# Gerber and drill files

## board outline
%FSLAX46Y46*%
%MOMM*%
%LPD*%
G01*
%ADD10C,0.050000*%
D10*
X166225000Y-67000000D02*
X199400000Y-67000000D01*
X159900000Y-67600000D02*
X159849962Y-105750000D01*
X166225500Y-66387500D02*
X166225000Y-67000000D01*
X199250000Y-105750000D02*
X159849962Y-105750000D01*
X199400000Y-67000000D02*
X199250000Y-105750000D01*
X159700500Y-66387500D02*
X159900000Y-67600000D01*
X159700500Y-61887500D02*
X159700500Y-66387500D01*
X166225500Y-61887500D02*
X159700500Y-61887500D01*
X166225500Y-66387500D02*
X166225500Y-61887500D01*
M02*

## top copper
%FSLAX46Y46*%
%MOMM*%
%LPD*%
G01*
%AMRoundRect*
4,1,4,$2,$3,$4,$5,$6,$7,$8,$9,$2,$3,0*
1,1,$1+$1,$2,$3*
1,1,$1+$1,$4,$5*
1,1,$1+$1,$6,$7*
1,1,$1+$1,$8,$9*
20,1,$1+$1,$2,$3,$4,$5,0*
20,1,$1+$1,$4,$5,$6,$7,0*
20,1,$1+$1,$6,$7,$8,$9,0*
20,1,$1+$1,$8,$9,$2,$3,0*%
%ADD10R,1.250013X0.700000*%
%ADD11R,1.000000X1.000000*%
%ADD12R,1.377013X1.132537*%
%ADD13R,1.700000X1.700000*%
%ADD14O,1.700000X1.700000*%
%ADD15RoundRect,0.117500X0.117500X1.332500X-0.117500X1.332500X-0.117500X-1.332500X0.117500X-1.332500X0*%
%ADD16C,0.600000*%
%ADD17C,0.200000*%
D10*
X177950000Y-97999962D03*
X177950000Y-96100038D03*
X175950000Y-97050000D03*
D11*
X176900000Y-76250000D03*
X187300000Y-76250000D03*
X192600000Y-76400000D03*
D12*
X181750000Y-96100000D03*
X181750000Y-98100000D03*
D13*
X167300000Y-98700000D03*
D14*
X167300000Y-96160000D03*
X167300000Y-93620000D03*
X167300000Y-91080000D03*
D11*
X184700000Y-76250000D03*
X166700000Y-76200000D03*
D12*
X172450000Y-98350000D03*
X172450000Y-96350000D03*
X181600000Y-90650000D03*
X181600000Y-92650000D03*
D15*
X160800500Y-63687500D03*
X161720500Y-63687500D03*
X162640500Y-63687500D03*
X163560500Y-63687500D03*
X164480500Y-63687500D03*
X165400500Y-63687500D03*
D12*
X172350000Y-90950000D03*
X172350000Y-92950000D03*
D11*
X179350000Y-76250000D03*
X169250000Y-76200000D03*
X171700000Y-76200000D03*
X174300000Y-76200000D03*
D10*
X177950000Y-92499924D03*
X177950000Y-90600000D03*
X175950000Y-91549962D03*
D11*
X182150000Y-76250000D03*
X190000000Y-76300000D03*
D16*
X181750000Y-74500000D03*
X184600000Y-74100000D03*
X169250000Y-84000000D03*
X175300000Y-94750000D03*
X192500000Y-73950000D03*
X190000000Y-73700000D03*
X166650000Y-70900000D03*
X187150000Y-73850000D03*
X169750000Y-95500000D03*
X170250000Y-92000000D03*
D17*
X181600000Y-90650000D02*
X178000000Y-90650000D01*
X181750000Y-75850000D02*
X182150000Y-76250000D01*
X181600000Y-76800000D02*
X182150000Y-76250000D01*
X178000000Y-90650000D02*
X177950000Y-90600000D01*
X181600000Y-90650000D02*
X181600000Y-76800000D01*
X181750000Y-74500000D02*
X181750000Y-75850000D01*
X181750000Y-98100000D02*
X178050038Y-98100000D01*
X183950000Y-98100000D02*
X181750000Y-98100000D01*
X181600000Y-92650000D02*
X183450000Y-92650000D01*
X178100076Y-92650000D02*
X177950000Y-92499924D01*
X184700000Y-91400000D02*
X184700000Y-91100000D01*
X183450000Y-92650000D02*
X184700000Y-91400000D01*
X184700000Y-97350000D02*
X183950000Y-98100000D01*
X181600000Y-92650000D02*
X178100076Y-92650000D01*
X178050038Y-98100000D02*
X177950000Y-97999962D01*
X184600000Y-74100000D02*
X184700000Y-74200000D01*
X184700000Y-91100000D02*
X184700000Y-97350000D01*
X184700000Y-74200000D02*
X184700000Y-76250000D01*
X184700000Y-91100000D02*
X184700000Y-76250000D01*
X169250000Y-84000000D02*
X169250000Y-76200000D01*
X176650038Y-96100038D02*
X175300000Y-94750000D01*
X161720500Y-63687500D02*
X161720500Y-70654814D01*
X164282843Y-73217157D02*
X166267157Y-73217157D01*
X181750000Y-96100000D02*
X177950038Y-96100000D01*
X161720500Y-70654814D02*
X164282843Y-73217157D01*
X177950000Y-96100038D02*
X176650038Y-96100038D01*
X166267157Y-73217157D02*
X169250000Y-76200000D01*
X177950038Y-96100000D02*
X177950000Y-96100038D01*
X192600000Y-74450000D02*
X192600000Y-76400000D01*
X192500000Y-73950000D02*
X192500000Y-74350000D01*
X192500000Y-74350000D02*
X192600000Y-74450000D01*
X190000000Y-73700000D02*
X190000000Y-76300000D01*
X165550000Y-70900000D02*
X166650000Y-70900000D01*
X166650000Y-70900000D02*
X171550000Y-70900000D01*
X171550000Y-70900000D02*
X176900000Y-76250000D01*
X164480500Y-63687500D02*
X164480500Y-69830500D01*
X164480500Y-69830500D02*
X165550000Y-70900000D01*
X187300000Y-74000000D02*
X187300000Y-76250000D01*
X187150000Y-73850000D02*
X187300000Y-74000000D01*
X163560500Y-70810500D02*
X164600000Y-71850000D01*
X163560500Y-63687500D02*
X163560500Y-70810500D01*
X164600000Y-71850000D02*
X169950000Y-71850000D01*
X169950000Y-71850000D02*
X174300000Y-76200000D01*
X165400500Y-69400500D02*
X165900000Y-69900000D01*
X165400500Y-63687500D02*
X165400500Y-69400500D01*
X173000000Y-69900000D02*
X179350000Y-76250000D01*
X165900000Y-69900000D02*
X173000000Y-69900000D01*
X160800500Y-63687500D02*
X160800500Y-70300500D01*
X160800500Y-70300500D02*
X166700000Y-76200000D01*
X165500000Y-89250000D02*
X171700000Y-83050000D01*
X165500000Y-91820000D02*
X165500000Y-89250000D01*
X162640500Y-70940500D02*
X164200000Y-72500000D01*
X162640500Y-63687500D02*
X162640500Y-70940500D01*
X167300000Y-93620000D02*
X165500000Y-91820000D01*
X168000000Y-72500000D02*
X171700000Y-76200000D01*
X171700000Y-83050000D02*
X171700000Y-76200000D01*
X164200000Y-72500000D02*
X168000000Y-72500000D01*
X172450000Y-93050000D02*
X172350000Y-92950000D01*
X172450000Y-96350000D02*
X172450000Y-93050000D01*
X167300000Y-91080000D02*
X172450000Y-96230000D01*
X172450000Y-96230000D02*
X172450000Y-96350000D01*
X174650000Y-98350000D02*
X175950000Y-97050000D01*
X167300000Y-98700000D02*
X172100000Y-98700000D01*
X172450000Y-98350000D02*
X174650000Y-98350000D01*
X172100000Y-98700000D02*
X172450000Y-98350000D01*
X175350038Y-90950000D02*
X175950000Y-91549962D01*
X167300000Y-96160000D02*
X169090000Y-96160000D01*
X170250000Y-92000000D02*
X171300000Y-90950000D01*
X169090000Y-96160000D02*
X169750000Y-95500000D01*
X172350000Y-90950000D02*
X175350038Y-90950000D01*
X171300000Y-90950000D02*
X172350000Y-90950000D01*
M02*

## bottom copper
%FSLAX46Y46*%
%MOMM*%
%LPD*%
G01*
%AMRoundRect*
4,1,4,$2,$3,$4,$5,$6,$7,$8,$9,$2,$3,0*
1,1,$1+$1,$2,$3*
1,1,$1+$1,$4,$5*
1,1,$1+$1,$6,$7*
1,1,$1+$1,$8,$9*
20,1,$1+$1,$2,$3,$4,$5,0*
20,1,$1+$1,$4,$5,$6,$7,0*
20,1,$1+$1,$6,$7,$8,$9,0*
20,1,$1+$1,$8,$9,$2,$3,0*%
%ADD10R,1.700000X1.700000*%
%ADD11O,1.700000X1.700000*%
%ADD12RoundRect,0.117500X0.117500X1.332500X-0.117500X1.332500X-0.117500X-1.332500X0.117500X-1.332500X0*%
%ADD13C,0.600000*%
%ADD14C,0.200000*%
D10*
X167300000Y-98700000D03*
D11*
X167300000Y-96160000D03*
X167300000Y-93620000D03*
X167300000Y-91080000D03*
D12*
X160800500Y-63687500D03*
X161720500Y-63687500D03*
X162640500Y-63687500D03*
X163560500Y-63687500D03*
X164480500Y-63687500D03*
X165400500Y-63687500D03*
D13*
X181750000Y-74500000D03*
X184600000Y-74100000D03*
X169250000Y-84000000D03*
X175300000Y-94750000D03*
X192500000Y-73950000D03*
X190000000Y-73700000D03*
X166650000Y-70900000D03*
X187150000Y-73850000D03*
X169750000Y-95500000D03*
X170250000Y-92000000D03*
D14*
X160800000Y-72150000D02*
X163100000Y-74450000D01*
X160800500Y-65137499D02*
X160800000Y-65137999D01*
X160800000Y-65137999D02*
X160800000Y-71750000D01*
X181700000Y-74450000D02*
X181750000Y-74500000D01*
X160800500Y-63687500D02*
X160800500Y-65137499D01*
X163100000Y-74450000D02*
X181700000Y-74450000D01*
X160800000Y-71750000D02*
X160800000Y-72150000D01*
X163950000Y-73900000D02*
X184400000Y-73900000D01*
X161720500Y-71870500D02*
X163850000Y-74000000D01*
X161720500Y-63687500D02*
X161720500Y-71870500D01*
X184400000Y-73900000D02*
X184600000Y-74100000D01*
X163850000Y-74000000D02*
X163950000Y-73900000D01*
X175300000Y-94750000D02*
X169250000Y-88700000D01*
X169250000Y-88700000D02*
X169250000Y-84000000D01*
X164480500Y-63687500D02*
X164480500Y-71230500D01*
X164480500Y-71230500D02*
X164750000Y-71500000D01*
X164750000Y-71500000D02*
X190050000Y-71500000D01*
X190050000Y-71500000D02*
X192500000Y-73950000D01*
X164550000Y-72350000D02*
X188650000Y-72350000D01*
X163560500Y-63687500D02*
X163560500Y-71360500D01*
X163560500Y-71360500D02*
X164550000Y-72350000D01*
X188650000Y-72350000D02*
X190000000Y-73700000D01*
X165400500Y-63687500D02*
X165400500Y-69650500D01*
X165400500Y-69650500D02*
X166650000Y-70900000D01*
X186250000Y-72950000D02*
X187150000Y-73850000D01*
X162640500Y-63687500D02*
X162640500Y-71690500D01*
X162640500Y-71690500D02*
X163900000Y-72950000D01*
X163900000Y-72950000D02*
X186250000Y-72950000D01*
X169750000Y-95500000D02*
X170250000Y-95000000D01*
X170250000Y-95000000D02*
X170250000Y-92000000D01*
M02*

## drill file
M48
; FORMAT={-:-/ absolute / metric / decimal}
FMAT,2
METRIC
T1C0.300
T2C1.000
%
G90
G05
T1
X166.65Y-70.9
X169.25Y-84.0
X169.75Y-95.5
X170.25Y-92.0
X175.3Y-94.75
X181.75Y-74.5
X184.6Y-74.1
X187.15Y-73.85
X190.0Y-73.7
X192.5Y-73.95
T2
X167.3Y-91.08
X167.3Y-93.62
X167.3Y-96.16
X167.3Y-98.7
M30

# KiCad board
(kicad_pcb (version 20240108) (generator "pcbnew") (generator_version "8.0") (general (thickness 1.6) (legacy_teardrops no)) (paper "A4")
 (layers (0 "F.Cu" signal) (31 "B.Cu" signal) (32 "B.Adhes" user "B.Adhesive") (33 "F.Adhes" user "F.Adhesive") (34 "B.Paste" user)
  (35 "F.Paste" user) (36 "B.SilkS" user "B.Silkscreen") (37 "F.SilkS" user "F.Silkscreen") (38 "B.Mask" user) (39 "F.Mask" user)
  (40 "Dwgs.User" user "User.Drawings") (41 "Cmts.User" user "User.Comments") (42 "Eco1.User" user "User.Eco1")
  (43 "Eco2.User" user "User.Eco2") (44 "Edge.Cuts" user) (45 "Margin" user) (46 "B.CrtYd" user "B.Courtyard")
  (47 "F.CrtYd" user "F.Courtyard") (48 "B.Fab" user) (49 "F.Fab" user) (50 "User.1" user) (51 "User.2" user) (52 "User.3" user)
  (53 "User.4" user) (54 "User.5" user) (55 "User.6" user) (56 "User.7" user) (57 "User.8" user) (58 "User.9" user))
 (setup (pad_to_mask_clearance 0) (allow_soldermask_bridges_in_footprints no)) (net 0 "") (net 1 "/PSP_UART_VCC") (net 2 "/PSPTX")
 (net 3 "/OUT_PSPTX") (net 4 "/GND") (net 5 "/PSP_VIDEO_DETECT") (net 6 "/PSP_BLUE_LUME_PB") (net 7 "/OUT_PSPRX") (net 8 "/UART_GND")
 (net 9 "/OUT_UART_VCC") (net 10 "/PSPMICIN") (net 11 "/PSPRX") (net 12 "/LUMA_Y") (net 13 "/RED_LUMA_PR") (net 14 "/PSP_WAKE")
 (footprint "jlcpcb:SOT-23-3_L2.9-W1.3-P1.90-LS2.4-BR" (layer "F.Cu") (at 176.95 97.05)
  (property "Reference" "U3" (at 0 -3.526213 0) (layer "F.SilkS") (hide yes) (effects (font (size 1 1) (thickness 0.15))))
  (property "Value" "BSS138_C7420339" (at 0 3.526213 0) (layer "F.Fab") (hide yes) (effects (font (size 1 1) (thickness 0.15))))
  (pad "1" smd rect (at 1 0.949962) (size 1.250013 0.7) (layers "F.Cu" "F.Paste" "F.Mask") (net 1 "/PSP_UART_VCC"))
  (pad "2" smd rect (at 1 -0.949962) (size 1.250013 0.7) (layers "F.Cu" "F.Paste" "F.Mask") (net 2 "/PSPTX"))
  (pad "3" smd rect (at -1 0) (size 1.250013 0.7) (layers "F.Cu" "F.Paste" "F.Mask") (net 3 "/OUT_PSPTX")))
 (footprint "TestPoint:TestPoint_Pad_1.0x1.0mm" (layer "F.Cu") (at 176.9 76.25)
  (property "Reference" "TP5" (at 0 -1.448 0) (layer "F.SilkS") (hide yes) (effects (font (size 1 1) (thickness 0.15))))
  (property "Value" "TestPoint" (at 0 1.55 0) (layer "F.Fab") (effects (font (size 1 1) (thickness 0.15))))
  (pad "1" smd rect (at 0 0) (size 1 1) (layers "F.Cu" "F.Mask") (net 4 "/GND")))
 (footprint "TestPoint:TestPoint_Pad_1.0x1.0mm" (layer "F.Cu") (at 187.3 76.25)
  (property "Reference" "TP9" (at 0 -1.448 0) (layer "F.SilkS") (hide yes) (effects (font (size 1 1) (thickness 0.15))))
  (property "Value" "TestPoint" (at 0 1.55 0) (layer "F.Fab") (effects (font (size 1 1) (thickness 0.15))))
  (pad "1" smd rect (at 0 0) (size 1 1) (layers "F.Cu" "F.Mask") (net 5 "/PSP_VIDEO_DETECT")))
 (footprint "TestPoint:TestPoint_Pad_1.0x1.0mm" (layer "F.Cu") (at 192.6 76.4)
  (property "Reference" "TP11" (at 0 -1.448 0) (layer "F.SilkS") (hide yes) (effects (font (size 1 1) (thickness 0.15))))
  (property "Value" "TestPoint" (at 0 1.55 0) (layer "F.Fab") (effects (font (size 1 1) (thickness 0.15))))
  (pad "1" smd rect (at 0 0) (size 1 1) (layers "F.Cu" "F.Mask") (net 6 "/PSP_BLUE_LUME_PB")))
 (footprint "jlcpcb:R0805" (layer "F.Cu") (at 181.75 97.1 -90)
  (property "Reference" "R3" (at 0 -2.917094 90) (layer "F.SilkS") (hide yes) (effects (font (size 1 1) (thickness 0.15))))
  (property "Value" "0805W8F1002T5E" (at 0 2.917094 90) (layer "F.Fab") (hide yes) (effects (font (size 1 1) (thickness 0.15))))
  (pad "1" smd rect (at -1 0 270) (size 1.132537 1.377013) (layers "F.Cu" "F.Paste" "F.Mask") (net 2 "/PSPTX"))
  (pad "2" smd rect (at 1 0 270) (size 1.132537 1.377013) (layers "F.Cu" "F.Paste" "F.Mask") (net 1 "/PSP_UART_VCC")))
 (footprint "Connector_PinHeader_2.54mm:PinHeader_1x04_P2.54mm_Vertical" (layer "F.Cu") (at 167.3 98.7 180)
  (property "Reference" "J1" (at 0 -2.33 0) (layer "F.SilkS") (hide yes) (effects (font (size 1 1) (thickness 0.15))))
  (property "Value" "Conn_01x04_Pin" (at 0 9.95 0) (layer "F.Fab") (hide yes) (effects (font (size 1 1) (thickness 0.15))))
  (pad "1" thru_hole rect (at 0 0 180) (size 1.7 1.7) (drill 1) (layers "*.Cu" "*.Mask") (remove_unused_layers no) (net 3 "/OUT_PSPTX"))
  (pad "2" thru_hole oval (at 0 2.54 180) (size 1.7 1.7) (drill 1) (layers "*.Cu" "*.Mask") (remove_unused_layers no) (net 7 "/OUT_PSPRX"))
  (pad "3" thru_hole oval (at 0 5.08 180) (size 1.7 1.7) (drill 1) (layers "*.Cu" "*.Mask") (remove_unused_layers no) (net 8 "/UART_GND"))
  (pad "4" thru_hole oval (at 0 7.62 180) (size 1.7 1.7) (drill 1) (layers "*.Cu" "*.Mask") (remove_unused_layers no)
   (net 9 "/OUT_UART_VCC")))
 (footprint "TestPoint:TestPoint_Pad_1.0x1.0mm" (layer "F.Cu") (at 184.7 76.25)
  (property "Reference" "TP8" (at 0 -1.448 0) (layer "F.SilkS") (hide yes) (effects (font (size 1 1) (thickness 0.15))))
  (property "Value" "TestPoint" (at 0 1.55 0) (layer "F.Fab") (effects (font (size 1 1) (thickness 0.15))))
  (pad "1" smd rect (at 0 0) (size 1 1) (layers "F.Cu" "F.Mask") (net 1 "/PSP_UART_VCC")))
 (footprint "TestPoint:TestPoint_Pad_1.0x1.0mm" (layer "F.Cu") (at 166.7 76.2)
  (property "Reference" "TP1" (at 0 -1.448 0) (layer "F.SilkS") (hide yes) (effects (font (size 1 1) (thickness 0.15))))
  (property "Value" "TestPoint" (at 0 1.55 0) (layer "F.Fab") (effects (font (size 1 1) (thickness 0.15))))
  (pad "1" smd rect (at 0 0) (size 1 1) (layers "F.Cu" "F.Mask") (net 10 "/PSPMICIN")))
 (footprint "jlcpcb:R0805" (layer "F.Cu") (at 172.45 97.35 90)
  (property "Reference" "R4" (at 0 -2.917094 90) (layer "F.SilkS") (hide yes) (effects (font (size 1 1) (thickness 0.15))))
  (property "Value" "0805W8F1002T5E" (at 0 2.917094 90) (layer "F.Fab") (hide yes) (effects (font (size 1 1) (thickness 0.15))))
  (pad "1" smd rect (at -1 0 90) (size 1.132537 1.377013) (layers "F.Cu" "F.Paste" "F.Mask") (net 3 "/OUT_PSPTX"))
  (pad "2" smd rect (at 1 0 90) (size 1.132537 1.377013) (layers "F.Cu" "F.Paste" "F.Mask") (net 9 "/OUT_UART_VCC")))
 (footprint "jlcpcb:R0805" (layer "F.Cu") (at 181.6 91.65 -90)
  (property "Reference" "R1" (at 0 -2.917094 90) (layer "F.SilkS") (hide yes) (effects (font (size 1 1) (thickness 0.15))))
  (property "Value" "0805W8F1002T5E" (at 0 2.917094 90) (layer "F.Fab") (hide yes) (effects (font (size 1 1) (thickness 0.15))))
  (pad "1" smd rect (at -1 0 270) (size 1.132537 1.377013) (layers "F.Cu" "F.Paste" "F.Mask") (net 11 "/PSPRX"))
  (pad "2" smd rect (at 1 0 270) (size 1.132537 1.377013) (layers "F.Cu" "F.Paste" "F.Mask") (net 1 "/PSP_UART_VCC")))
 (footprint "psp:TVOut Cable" (layer "F.Cu") (at 168.8255 70.9875)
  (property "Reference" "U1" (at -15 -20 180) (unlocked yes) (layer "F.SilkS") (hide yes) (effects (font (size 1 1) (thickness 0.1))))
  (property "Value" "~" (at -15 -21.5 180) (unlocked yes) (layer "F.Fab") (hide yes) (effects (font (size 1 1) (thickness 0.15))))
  (fp_line (start -9.125 -9.1) (end -9.125 -4.6) (stroke (width 0.05) (type default)) (layer "Edge.Cuts"))
  (fp_line (start -2.6 -9.1) (end -9.125 -9.1) (stroke (width 0.05) (type default)) (layer "Edge.Cuts"))
  (fp_line (start -2.6 -4.6) (end -2.6 -9.1) (stroke (width 0.05) (type default)) (layer "Edge.Cuts"))
  (pad "1" smd roundrect (at -8.025 -7.3 180) (size 0.47 2.9) (layers "F.Cu" "F.Paste" "F.Mask") (roundrect_rratio 0.25)
   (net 10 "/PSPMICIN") (thermal_bridge_angle 45))
  (pad "2" smd roundrect (at -7.105 -7.3 180) (size 0.47 2.9) (layers "F.Cu" "F.Paste" "F.Mask") (roundrect_rratio 0.25) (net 2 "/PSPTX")
   (thermal_bridge_angle 45))
  (pad "3" smd roundrect (at -6.185 -7.3 180) (size 0.47 2.9) (layers "F.Cu" "F.Paste" "F.Mask") (roundrect_rratio 0.25) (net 8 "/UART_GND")
   (thermal_bridge_angle 45))
  (pad "4" smd roundrect (at -5.265 -7.3 180) (size 0.47 2.9) (layers "F.Cu" "F.Paste" "F.Mask") (roundrect_rratio 0.25) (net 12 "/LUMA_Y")
   (thermal_bridge_angle 45))
  (pad "5" smd roundrect (at -4.345 -7.3 180) (size 0.47 2.9) (layers "F.Cu" "F.Paste" "F.Mask") (roundrect_rratio 0.25) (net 4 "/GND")
   (thermal_bridge_angle 45))
  (pad "6" smd roundrect (at -3.425 -7.3 180) (size 0.47 2.9) (layers "F.Cu" "F.Paste" "F.Mask") (roundrect_rratio 0.25)
   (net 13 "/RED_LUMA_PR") (thermal_bridge_angle 45))
  (pad "7" smd roundrect (at -8.025 -7.3 180) (size 0.47 2.9) (layers "B.Cu" "B.Paste" "B.Mask") (roundrect_rratio 0.25) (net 11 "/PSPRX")
   (thermal_bridge_angle 45))
  (pad "8" smd roundrect (at -7.105 -7.3 180) (size 0.47 2.9) (layers "B.Cu" "B.Paste" "B.Mask") (roundrect_rratio 0.25)
   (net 1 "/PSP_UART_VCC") (thermal_bridge_angle 45))
  (pad "9" smd roundrect (at -6.185 -7.3 180) (size 0.47 2.9) (layers "B.Cu" "B.Paste" "B.Mask") (roundrect_rratio 0.25)
   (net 5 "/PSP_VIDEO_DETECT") (thermal_bridge_angle 45))
  (pad "10" smd roundrect (at -5.265 -7.3 180) (size 0.47 2.9) (layers "B.Cu" "B.Paste" "B.Mask") (roundrect_rratio 0.25)
   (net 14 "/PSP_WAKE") (thermal_bridge_angle 45))
  (pad "11" smd roundrect (at -4.345 -7.3 180) (size 0.47 2.9) (layers "B.Cu" "B.Paste" "B.Mask") (roundrect_rratio 0.25)
   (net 6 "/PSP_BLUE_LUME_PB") (thermal_bridge_angle 45))
  (pad "12" smd roundrect (at -3.425 -7.3 180) (size 0.47 2.9) (layers "B.Cu" "B.Paste" "B.Mask") (roundrect_rratio 0.25) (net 4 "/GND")
   (thermal_bridge_angle 45)))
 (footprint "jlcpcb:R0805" (layer "F.Cu") (at 172.35 91.95 -90)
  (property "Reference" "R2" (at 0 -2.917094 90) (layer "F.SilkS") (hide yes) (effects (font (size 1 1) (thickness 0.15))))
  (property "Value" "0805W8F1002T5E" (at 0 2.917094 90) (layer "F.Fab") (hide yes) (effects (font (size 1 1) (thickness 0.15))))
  (pad "1" smd rect (at -1 0 270) (size 1.132537 1.377013) (layers "F.Cu" "F.Paste" "F.Mask") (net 7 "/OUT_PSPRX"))
  (pad "2" smd rect (at 1 0 270) (size 1.132537 1.377013) (layers "F.Cu" "F.Paste" "F.Mask") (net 9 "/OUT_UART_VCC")))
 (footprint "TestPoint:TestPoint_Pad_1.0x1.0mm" (layer "F.Cu") (at 179.35 76.25)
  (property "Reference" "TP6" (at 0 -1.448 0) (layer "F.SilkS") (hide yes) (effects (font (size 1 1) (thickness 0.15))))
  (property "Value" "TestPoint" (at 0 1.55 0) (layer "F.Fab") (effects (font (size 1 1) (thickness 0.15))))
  (pad "1" smd rect (at 0 0) (size 1 1) (layers "F.Cu" "F.Mask") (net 13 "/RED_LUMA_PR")))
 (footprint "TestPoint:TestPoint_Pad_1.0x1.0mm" (layer "F.Cu") (at 169.25 76.2)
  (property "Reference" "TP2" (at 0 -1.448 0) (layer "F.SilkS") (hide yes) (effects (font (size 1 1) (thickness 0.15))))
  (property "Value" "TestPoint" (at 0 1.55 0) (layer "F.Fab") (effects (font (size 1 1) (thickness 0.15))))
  (pad "1" smd rect (at 0 0) (size 1 1) (layers "F.Cu" "F.Mask") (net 2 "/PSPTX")))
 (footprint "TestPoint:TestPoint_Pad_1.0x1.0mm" (layer "F.Cu") (at 171.7 76.2)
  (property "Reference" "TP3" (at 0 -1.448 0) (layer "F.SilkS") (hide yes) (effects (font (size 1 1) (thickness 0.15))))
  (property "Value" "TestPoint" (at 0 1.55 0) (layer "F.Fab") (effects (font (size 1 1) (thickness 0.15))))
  (pad "1" smd rect (at 0 0) (size 1 1) (layers "F.Cu" "F.Mask") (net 8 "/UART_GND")))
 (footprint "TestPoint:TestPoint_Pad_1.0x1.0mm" (layer "F.Cu") (at 174.3 76.2)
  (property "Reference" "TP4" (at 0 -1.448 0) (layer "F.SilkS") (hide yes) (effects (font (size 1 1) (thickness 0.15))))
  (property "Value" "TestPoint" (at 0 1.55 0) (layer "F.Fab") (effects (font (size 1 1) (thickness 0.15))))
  (pad "1" smd rect (at 0 0) (size 1 1) (layers "F.Cu" "F.Mask") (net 12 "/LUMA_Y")))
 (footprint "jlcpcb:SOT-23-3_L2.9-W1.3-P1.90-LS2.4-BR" (layer "F.Cu") (at 176.95 91.549962)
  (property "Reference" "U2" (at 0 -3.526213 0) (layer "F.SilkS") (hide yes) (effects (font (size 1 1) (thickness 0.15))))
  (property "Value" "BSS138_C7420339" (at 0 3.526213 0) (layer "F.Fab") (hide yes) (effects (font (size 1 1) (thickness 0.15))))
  (pad "1" smd rect (at 1 0.949962) (size 1.250013 0.7) (layers "F.Cu" "F.Paste" "F.Mask") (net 1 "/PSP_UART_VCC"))
  (pad "2" smd rect (at 1 -0.949962) (size 1.250013 0.7) (layers "F.Cu" "F.Paste" "F.Mask") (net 11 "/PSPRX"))
  (pad "3" smd rect (at -1 0) (size 1.250013 0.7) (layers "F.Cu" "F.Paste" "F.Mask") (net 7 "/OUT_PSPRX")))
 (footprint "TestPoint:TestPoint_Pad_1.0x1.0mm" (layer "F.Cu") (at 182.15 76.25)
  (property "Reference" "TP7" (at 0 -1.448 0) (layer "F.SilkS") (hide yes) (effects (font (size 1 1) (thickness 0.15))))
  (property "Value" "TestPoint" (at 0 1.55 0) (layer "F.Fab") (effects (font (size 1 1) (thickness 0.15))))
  (pad "1" smd rect (at 0 0) (size 1 1) (layers "F.Cu" "F.Mask") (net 11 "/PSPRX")))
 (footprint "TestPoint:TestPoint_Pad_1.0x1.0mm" (layer "F.Cu") (at 190 76.3)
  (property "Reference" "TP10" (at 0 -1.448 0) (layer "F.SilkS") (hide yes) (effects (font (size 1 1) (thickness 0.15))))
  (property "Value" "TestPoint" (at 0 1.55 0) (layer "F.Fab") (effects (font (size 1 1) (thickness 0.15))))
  (pad "1" smd rect (at 0 0) (size 1 1) (layers "F.Cu" "F.Mask") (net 14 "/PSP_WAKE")))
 (gr_line (start 166.225 67) (end 199.4 67) (stroke (width 0.05) (type default)) (layer "Edge.Cuts"))
 (gr_line (start 159.9 67.6) (end 159.849962 105.75) (stroke (width 0.05) (type default)) (layer "Edge.Cuts"))
 (gr_line (start 166.2255 66.3875) (end 166.225 67) (stroke (width 0.05) (type default)) (layer "Edge.Cuts"))
 (gr_line (start 199.25 105.75) (end 159.849962 105.75) (stroke (width 0.05) (type default)) (layer "Edge.Cuts"))
 (gr_line (start 199.4 67) (end 199.25 105.75) (stroke (width 0.05) (type default)) (layer "Edge.Cuts"))
 (gr_line (start 159.7005 66.3875) (end 159.9 67.6) (stroke (width 0.05) (type default)) (layer "Edge.Cuts"))
 (segment (start 181.6 90.65) (end 178 90.65) (width 0.2) (layer "F.Cu") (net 11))
 (segment (start 181.75 75.85) (end 182.15 76.25) (width 0.2) (layer "F.Cu") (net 11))
 (segment (start 181.6 76.8) (end 182.15 76.25) (width 0.2) (layer "F.Cu") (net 11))
 (segment (start 178 90.65) (end 177.95 90.6) (width 0.2) (layer "F.Cu") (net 11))
 (segment (start 181.6 90.65) (end 181.6 76.8) (width 0.2) (layer "F.Cu") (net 11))
 (segment (start 181.75 74.5) (end 181.75 75.85) (width 0.2) (layer "F.Cu") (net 11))
 (via (at 181.75 74.5) (size 0.6) (drill 0.3) (layers "F.Cu" "B.Cu") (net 11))
 (segment (start 160.8 72.15) (end 163.1 74.45) (width 0.2) (layer "B.Cu") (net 11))
 (segment (start 160.8005 65.137499) (end 160.8 65.137999) (width 0.2) (layer "B.Cu") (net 11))
 (segment (start 160.8 65.137999) (end 160.8 71.75) (width 0.2) (layer "B.Cu") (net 11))
 (segment (start 181.7 74.45) (end 181.75 74.5) (width 0.2) (layer "B.Cu") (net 11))
 (segment (start 160.8005 63.6875) (end 160.8005 65.137499) (width 0.2) (layer "B.Cu") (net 11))
 (segment (start 163.1 74.45) (end 181.7 74.45) (width 0.2) (layer "B.Cu") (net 11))
 (segment (start 160.8 71.75) (end 160.8 72.15) (width 0.2) (layer "B.Cu") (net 11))
 (segment (start 181.75 98.1) (end 178.050038 98.1) (width 0.2) (layer "F.Cu") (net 1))
 (segment (start 183.95 98.1) (end 181.75 98.1) (width 0.2) (layer "F.Cu") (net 1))
 (segment (start 181.6 92.65) (end 183.45 92.65) (width 0.2) (layer "F.Cu") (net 1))
 (segment (start 178.100076 92.65) (end 177.95 92.499924) (width 0.2) (layer "F.Cu") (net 1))
 (segment (start 184.7 91.4) (end 184.7 91.1) (width 0.2) (layer "F.Cu") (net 1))
 (segment (start 183.45 92.65) (end 184.7 91.4) (width 0.2) (layer "F.Cu") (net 1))
 (segment (start 184.7 97.35) (end 183.95 98.1) (width 0.2) (layer "F.Cu") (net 1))
 (segment (start 181.6 92.65) (end 178.100076 92.65) (width 0.2) (layer "F.Cu") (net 1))
 (segment (start 178.050038 98.1) (end 177.95 97.999962) (width 0.2) (layer "F.Cu") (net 1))
 (segment (start 184.6 74.1) (end 184.7 74.2) (width 0.2) (layer "F.Cu") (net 1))
 (segment (start 184.7 91.1) (end 184.7 97.35) (width 0.2) (layer "F.Cu") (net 1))
 (segment (start 184.7 74.2) (end 184.7 76.25) (width 0.2) (layer "F.Cu") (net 1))
 (segment (start 184.7 91.1) (end 184.7 76.25) (width 0.2) (layer "F.Cu") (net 1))
 (via (at 184.6 74.1) (size 0.6) (drill 0.3) (layers "F.Cu" "B.Cu") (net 1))
 (segment (start 163.95 73.9) (end 184.4 73.9) (width 0.2) (layer "B.Cu") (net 1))
 (segment (start 161.7205 71.8705) (end 163.85 74) (width 0.2) (layer "B.Cu") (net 1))
 (segment (start 161.7205 63.6875) (end 161.7205 71.8705) (width 0.2) (layer "B.Cu") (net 1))
 (segment (start 184.4 73.9) (end 184.6 74.1) (width 0.2) (layer "B.Cu") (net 1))
 (segment (start 163.85 74) (end 163.95 73.9) (width 0.2) (layer "B.Cu") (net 1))
 (segment (start 169.25 84) (end 169.25 76.2) (width 0.2) (layer "F.Cu") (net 2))
 (segment (start 176.650038 96.100038) (end 175.3 94.75) (width 0.2) (layer "F.Cu") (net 2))
 (segment (start 161.7205 63.6875) (end 161.7205 70.654814) (width 0.2) (layer "F.Cu") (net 2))
 (segment (start 164.282843 73.217157) (end 166.267157 73.217157) (width 0.2) (layer "F.Cu") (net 2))
 (segment (start 181.75 96.1) (end 177.950038 96.1) (width 0.2) (layer "F.Cu") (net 2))
 (segment (start 161.7205 70.654814) (end 164.282843 73.217157) (width 0.2) (layer "F.Cu") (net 2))
 (segment (start 177.95 96.100038) (end 176.650038 96.100038) (width 0.2) (layer "F.Cu") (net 2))
 (segment (start 166.267157 73.217157) (end 169.25 76.2) (width 0.2) (layer "F.Cu") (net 2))
 (segment (start 177.950038 96.1) (end 177.95 96.100038) (width 0.2) (layer "F.Cu") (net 2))
 (via (at 169.25 84) (size 0.6) (drill 0.3) (layers "F.Cu" "B.Cu") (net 2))
 (via (at 175.3 94.75) (size 0.6) (drill 0.3) (layers "F.Cu" "B.Cu") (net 2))
 (segment (start 175.3 94.75) (end 169.25 88.7) (width 0.2) (layer "B.Cu") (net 2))
 (segment (start 169.25 88.7) (end 169.25 84) (width 0.2) (layer "B.Cu") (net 2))
 (segment (start 192.6 74.45) (end 192.6 76.4) (width 0.2) (layer "F.Cu") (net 6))
 (segment (start 192.5 73.95) (end 192.5 74.35) (width 0.2) (layer "F.Cu") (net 6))
 (segment (start 192.5 74.35) (end 192.6 74.45) (width 0.2) (layer "F.Cu") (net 6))
 (via (at 192.5 73.95) (size 0.6) (drill 0.3) (layers "F.Cu" "B.Cu") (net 6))
 (segment (start 164.4805 63.6875) (end 164.4805 71.2305) (width 0.2) (layer "B.Cu") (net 6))
 (segment (start 164.4805 71.2305) (end 164.75 71.5) (width 0.2) (layer "B.Cu") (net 6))
 (segment (start 164.75 71.5) (end 190.05 71.5) (width 0.2) (layer "B.Cu") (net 6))
 (segment (start 190.05 71.5) (end 192.5 73.95) (width 0.2) (layer "B.Cu") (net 6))
 (segment (start 190 73.7) (end 190 76.3) (width 0.2) (layer "F.Cu") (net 14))
 (via (at 190 73.7) (size 0.6) (drill 0.3) (layers "F.Cu" "B.Cu") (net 14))
 (segment (start 164.55 72.35) (end 188.65 72.35) (width 0.2) (layer "B.Cu") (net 14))
 (segment (start 163.5605 63.6875) (end 163.5605 71.3605) (width 0.2) (layer "B.Cu") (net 14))
 (segment (start 163.5605 71.3605) (end 164.55 72.35) (width 0.2) (layer "B.Cu") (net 14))
 (segment (start 188.65 72.35) (end 190 73.7) (width 0.2) (layer "B.Cu") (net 14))
 (segment (start 165.55 70.9) (end 166.65 70.9) (width 0.2) (layer "F.Cu") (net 4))
 (segment (start 166.65 70.9) (end 171.55 70.9) (width 0.2) (layer "F.Cu") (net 4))
 (segment (start 171.55 70.9) (end 176.9 76.25) (width 0.2) (layer "F.Cu") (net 4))
 (segment (start 164.4805 63.6875) (end 164.4805 69.8305) (width 0.2) (layer "F.Cu") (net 4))
 (segment (start 164.4805 69.8305) (end 165.55 70.9) (width 0.2) (layer "F.Cu") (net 4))
 (via (at 166.65 70.9) (size 0.6) (drill 0.3) (layers "F.Cu" "B.Cu") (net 4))
 (segment (start 165.4005 63.6875) (end 165.4005 69.6505) (width 0.2) (layer "B.Cu") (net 4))
 (segment (start 165.4005 69.6505) (end 166.65 70.9) (width 0.2) (layer "B.Cu") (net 4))
 (segment (start 187.3 74) (end 187.3 76.25) (width 0.2) (layer "F.Cu") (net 5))
 (segment (start 187.15 73.85) (end 187.3 74) (width 0.2) (layer "F.Cu") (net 5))
 (via (at 187.15 73.85) (size 0.6) (drill 0.3) (layers "F.Cu" "B.Cu") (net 5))
 (segment (start 186.25 72.95) (end 187.15 73.85) (width 0.2) (layer "B.Cu") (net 5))
 (segment (start 162.6405 63.6875) (end 162.6405 71.6905) (width 0.2) (layer "B.Cu") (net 5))
 (segment (start 162.6405 71.6905) (end 163.9 72.95) (width 0.2) (layer "B.Cu") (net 5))
 (segment (start 163.9 72.95) (end 186.25 72.95) (width 0.2) (layer "B.Cu") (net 5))
 (segment (start 163.5605 70.8105) (end 164.6 71.85) (width 0.2) (layer "F.Cu") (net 12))
 (segment (start 163.5605 63.6875) (end 163.5605 70.8105) (width 0.2) (layer "F.Cu") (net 12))
 (segment (start 164.6 71.85) (end 169.95 71.85) (width 0.2) (layer "F.Cu") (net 12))
 (segment (start 169.95 71.85) (end 174.3 76.2) (width 0.2) (layer "F.Cu") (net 12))
 (segment (start 165.4005 69.4005) (end 165.9 69.9) (width 0.2) (layer "F.Cu") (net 13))
 (segment (start 165.4005 63.6875) (end 165.4005 69.4005) (width 0.2) (layer "F.Cu") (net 13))
 (segment (start 173 69.9) (end 179.35 76.25) (width 0.2) (layer "F.Cu") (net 13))
 (segment (start 165.9 69.9) (end 173 69.9) (width 0.2) (layer "F.Cu") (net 13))
 (segment (start 160.8005 63.6875) (end 160.8005 70.3005) (width 0.2) (layer "F.Cu") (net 10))
 (segment (start 160.8005 70.3005) (end 166.7 76.2) (width 0.2) (layer "F.Cu") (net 10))
 (segment (start 165.5 89.25) (end 171.7 83.05) (width 0.2) (layer "F.Cu") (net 8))
 (segment (start 165.5 91.82) (end 165.5 89.25) (width 0.2) (layer "F.Cu") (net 8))
 (segment (start 162.6405 70.9405) (end 164.2 72.5) (width 0.2) (layer "F.Cu") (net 8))
 (segment (start 162.6405 63.6875) (end 162.6405 70.9405) (width 0.2) (layer "F.Cu") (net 8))
 (segment (start 167.3 93.62) (end 165.5 91.82) (width 0.2) (layer "F.Cu") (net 8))
 (segment (start 168 72.5) (end 171.7 76.2) (width 0.2) (layer "F.Cu") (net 8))
 (segment (start 171.7 83.05) (end 171.7 76.2) (width 0.2) (layer "F.Cu") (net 8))
 (segment (start 164.2 72.5) (end 168 72.5) (width 0.2) (layer "F.Cu") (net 8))
 (segment (start 172.45 93.05) (end 172.35 92.95) (width 0.2) (layer "F.Cu") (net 9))
 (segment (start 172.45 96.35) (end 172.45 93.05) (width 0.2) (layer "F.Cu") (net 9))
 (segment (start 167.3 91.08) (end 172.45 96.23) (width 0.2) (layer "F.Cu") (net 9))
 (segment (start 172.45 96.23) (end 172.45 96.35) (width 0.2) (layer "F.Cu") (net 9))
 (segment (start 174.65 98.35) (end 175.95 97.05) (width 0.2) (layer "F.Cu") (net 3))
 (segment (start 167.3 98.7) (end 172.1 98.7) (width 0.2) (layer "F.Cu") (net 3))
 (segment (start 172.45 98.35) (end 174.65 98.35) (width 0.2) (layer "F.Cu") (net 3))
 (segment (start 172.1 98.7) (end 172.45 98.35) (width 0.2) (layer "F.Cu") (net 3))
 (segment (start 175.350038 90.95) (end 175.95 91.549962) (width 0.2) (layer "F.Cu") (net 7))
 (segment (start 167.3 96.16) (end 169.09 96.16) (width 0.2) (layer "F.Cu") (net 7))
 (segment (start 170.25 92) (end 171.3 90.95) (width 0.2) (layer "F.Cu") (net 7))
 (segment (start 169.09 96.16) (end 169.75 95.5) (width 0.2) (layer "F.Cu") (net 7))
 (segment (start 172.35 90.95) (end 175.350038 90.95) (width 0.2) (layer "F.Cu") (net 7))
 (segment (start 171.3 90.95) (end 172.35 90.95) (width 0.2) (layer "F.Cu") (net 7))
 (via (at 169.75 95.5) (size 0.6) (drill 0.3) (layers "F.Cu" "B.Cu") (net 7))
 (via (at 170.25 92) (size 0.6) (drill 0.3) (layers "F.Cu" "B.Cu") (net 7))
 (segment (start 169.75 95.5) (end 170.25 95) (width 0.2) (layer "B.Cu") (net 7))
 (segment (start 170.25 95) (end 170.25 92) (width 0.2) (layer "B.Cu") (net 7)))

